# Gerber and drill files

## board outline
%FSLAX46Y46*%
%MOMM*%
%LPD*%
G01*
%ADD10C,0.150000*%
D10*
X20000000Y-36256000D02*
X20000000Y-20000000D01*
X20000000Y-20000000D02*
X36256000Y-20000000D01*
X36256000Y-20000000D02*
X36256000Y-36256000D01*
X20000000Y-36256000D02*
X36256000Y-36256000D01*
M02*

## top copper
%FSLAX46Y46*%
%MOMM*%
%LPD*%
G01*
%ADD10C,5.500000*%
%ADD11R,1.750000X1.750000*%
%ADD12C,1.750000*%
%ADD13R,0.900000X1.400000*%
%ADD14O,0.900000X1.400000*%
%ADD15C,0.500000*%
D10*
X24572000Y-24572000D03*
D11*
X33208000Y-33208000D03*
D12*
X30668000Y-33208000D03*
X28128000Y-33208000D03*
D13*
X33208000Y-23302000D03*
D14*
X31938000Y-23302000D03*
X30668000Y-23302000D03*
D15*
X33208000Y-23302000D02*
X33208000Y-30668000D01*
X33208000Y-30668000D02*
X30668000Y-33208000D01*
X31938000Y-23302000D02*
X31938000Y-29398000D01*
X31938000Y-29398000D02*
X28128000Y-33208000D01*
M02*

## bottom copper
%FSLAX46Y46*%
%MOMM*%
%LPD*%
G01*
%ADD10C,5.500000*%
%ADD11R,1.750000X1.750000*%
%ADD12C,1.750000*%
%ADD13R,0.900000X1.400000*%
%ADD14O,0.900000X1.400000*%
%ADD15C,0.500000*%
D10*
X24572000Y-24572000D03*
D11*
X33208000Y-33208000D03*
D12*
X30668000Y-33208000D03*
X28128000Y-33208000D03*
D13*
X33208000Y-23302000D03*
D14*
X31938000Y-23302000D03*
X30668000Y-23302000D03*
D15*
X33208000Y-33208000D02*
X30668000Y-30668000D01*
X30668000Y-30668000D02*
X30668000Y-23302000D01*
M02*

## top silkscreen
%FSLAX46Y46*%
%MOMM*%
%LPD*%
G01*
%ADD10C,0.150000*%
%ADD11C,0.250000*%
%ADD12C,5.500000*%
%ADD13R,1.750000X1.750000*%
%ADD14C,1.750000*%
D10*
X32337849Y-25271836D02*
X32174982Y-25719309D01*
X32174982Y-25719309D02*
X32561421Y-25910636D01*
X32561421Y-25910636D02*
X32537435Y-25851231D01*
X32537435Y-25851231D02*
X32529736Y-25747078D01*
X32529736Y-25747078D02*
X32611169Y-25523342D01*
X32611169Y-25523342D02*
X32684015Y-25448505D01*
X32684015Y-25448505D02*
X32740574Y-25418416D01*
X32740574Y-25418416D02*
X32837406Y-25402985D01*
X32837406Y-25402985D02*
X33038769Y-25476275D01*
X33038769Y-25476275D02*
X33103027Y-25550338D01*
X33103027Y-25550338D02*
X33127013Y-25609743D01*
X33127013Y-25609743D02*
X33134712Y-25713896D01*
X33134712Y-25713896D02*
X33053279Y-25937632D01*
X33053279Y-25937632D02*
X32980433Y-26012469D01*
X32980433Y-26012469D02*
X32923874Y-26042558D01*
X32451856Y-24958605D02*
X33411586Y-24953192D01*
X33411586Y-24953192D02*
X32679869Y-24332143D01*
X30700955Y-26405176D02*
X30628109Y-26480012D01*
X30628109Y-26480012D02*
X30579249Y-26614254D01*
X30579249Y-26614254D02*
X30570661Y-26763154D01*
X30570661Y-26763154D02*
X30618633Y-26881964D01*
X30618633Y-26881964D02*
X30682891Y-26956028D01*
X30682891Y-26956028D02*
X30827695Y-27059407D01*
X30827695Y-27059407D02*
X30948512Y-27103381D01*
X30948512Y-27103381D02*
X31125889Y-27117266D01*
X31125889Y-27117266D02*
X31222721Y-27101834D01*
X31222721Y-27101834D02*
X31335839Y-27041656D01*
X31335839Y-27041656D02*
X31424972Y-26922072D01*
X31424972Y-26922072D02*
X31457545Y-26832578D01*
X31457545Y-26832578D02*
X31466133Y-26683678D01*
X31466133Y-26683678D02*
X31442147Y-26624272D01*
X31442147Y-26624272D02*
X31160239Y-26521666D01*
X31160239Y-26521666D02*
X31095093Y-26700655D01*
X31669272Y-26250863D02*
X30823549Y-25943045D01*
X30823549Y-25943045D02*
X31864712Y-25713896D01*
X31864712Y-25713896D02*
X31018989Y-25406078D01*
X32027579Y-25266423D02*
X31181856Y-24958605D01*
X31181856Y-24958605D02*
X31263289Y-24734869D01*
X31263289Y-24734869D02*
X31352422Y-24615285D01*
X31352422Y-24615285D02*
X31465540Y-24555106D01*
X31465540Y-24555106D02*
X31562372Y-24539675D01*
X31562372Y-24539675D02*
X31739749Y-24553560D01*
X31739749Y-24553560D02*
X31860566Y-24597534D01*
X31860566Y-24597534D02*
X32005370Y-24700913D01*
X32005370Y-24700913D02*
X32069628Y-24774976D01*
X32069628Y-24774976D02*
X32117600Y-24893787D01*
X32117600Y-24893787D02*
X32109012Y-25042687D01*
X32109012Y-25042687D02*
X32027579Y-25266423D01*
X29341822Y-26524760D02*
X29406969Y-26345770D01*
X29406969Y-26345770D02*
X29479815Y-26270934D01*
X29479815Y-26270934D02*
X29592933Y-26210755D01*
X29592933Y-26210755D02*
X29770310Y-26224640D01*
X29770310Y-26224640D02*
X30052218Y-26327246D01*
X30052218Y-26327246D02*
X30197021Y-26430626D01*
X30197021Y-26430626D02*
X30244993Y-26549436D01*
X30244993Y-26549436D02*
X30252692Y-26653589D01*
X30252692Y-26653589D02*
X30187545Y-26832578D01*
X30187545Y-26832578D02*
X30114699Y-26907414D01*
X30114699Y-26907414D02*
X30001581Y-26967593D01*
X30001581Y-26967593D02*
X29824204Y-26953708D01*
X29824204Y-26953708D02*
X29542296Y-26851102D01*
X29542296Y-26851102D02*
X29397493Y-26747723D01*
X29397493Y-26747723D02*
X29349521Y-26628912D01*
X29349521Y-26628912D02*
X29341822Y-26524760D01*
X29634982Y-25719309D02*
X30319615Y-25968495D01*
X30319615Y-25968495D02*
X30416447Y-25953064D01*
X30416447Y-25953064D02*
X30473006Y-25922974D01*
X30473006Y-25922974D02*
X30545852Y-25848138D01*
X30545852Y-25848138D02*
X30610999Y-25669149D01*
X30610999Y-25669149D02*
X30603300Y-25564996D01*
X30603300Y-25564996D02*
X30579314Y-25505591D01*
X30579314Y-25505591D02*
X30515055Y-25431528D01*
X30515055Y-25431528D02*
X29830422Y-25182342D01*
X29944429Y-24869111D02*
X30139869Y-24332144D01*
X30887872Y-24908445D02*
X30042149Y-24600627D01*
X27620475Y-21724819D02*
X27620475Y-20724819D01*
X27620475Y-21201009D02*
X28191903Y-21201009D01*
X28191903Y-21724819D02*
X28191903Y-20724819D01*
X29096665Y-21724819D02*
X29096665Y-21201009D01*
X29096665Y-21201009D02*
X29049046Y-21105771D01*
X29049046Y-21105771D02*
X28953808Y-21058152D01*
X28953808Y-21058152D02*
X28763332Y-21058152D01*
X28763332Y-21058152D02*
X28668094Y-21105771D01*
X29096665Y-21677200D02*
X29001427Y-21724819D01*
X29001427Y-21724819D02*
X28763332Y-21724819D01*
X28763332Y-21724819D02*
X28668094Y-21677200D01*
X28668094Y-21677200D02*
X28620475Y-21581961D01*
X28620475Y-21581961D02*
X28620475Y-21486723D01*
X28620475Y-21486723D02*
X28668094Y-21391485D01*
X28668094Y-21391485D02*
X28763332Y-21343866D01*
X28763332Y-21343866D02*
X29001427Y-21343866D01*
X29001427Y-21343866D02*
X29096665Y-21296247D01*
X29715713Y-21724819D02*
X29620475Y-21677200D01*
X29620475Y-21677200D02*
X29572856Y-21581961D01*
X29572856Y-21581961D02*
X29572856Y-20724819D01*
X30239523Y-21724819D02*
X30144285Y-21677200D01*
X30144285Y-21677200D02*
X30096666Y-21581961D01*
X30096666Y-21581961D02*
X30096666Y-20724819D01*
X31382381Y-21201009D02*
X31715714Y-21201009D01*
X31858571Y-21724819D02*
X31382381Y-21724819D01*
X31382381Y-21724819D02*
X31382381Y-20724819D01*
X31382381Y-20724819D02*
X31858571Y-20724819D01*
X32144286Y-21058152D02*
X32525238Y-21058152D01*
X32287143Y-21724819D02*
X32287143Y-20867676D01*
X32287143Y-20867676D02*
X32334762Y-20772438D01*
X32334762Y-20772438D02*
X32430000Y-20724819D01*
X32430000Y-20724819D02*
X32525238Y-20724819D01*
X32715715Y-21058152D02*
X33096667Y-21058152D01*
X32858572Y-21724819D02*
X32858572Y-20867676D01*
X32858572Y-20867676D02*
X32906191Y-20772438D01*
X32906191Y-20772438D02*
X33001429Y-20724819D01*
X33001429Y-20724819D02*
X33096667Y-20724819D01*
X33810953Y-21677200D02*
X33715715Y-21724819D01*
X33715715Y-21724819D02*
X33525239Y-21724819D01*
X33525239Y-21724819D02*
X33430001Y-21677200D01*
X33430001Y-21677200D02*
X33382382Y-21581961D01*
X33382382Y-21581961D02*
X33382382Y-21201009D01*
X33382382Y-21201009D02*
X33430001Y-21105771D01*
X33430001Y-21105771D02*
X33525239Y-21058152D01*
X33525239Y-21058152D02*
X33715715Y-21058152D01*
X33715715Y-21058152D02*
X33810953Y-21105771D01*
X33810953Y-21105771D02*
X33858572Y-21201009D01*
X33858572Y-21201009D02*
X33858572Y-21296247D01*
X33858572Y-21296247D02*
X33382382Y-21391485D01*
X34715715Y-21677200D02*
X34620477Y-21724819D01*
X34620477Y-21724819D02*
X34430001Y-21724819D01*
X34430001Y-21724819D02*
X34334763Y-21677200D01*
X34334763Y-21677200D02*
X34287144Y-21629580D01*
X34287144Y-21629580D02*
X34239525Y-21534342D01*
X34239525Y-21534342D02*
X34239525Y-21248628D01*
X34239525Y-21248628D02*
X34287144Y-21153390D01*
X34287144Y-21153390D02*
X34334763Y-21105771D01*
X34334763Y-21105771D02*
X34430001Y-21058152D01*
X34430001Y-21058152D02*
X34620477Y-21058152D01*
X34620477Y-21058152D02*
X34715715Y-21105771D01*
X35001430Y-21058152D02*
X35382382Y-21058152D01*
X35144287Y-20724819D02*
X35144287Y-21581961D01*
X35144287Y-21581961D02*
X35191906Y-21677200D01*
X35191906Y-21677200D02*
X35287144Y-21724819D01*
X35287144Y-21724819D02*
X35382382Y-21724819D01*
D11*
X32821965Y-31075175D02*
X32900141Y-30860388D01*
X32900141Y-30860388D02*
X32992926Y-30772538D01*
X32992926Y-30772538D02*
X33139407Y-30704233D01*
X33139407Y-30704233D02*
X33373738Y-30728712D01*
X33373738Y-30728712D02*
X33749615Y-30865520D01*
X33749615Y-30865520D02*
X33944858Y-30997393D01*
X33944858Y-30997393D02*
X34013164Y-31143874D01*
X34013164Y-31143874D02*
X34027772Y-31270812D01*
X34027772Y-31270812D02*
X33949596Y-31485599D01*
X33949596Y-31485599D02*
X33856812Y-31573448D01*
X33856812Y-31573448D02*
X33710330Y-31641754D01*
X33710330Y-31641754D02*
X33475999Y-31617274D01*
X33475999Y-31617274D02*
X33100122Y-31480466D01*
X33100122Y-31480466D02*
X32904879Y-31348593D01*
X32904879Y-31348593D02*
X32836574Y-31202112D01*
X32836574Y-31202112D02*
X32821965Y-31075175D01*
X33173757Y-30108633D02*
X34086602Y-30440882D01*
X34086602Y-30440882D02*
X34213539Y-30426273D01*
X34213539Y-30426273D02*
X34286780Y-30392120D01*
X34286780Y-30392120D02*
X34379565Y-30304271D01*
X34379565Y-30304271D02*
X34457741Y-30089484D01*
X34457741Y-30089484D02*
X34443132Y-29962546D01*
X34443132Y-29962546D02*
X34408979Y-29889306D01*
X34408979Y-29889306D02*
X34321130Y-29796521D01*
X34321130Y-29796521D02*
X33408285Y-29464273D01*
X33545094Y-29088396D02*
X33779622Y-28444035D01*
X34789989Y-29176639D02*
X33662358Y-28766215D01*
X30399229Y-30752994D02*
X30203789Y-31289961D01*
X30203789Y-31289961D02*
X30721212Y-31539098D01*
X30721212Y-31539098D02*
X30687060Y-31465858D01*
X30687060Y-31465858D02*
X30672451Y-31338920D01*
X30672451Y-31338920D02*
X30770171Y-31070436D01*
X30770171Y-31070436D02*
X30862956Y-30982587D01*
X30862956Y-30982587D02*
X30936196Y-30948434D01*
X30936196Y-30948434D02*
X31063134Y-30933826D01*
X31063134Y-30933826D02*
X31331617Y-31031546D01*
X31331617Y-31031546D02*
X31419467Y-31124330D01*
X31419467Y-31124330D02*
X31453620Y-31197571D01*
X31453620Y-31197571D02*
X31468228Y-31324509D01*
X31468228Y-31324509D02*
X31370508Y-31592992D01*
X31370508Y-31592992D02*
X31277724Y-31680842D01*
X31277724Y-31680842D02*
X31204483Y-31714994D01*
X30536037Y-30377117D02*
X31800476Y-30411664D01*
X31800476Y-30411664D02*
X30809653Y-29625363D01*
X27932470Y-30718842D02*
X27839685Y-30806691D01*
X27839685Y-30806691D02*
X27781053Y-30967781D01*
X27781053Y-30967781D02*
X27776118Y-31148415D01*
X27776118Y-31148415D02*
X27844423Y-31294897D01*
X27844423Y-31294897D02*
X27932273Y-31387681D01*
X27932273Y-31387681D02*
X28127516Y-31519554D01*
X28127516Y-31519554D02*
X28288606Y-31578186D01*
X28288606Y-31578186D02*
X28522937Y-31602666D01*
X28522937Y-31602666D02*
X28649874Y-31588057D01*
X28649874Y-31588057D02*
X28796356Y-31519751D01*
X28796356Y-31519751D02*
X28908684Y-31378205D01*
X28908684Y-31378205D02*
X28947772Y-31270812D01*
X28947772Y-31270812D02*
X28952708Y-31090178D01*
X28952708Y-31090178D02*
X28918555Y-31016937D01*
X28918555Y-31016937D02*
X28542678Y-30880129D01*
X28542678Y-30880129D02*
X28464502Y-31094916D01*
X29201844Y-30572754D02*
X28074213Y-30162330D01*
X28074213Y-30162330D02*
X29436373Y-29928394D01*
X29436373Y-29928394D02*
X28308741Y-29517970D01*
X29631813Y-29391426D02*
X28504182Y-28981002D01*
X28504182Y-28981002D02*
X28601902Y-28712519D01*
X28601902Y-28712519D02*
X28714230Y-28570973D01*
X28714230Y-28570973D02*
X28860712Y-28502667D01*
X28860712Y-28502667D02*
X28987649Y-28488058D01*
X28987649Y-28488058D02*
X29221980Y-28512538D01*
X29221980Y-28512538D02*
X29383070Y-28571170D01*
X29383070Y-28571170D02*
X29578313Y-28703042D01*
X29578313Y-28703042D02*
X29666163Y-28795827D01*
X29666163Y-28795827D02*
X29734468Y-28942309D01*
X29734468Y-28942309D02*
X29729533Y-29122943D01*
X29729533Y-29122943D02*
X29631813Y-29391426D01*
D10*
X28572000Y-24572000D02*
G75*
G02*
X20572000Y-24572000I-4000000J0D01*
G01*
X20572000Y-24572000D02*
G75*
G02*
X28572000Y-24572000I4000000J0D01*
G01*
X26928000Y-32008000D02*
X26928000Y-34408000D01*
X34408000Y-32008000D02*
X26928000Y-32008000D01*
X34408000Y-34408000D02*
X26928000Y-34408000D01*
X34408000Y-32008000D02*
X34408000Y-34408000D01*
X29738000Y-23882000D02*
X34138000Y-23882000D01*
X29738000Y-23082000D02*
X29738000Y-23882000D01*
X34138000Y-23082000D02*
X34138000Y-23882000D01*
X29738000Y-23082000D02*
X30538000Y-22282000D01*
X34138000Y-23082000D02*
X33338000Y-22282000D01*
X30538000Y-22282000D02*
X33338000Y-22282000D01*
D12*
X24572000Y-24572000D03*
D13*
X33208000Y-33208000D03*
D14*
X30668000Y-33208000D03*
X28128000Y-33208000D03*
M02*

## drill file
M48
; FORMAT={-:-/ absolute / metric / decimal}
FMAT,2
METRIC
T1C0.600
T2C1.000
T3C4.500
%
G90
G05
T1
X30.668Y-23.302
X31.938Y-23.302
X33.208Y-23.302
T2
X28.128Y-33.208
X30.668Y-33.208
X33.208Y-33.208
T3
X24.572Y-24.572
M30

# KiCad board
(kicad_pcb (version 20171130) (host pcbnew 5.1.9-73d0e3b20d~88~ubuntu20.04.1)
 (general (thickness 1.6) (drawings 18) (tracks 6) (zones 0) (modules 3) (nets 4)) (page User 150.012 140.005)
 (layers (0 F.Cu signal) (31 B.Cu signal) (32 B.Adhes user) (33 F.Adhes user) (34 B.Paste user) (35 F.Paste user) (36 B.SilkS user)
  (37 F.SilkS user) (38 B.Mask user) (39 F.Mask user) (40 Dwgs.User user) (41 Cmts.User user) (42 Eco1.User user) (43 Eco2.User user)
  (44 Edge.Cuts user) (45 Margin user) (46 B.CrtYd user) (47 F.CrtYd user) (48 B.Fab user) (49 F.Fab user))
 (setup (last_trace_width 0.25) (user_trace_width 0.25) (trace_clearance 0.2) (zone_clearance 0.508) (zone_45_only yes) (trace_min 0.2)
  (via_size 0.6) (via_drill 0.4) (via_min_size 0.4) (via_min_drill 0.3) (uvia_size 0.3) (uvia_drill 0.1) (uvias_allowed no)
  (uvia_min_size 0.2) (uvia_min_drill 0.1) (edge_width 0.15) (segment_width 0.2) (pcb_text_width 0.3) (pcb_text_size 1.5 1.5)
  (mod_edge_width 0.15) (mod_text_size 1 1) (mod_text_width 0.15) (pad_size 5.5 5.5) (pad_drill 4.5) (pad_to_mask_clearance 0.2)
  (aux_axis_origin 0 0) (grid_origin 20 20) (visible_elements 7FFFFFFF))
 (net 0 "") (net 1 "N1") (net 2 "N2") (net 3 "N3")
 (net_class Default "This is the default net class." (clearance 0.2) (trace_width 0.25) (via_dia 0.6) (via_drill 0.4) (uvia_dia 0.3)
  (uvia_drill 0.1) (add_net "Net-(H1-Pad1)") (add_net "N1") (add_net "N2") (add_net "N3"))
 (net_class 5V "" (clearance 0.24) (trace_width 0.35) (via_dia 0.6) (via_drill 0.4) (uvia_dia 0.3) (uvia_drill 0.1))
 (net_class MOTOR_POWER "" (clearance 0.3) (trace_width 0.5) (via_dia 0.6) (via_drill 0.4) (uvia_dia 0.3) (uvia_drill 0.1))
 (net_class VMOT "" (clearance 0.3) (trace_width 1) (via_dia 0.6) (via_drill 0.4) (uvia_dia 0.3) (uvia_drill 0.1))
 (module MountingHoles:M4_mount (layer F.Cu) (at 24.572 24.572)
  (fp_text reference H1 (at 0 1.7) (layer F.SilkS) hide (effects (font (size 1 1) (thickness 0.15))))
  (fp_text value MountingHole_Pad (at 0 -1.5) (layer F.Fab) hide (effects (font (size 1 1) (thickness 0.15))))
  (fp_circle (center 0 0) (end 4 0) (layer F.SilkS) (width 0.15))
  (pad 1 thru_hole circle (at 0 0) (size 5.5 5.5) (drill 4.5) (layers *.Cu *.Mask F.SilkS) (clearance 1.5)))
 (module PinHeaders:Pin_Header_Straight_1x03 (layer F.Cu) (at 33.208 33.208 270)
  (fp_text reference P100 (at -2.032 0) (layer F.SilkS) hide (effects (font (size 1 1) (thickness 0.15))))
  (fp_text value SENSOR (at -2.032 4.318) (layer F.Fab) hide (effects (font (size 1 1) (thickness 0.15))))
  (fp_line (start -1.2 6.28) (end 1.2 6.28) (layer F.SilkS) (width 0.15))
  (fp_line (start -1.2 -1.2) (end -1.2 6.28) (layer F.SilkS) (width 0.15))
  (fp_line (start 1.2 -1.2) (end 1.2 6.28) (layer F.SilkS) (width 0.15))
  (fp_line (start -1.2 -1.2) (end 1.2 -1.2) (layer F.SilkS) (width 0.15))
  (pad 1 thru_hole rect (at 0 0 270) (size 1.75 1.75) (drill 1) (layers *.Cu *.Mask F.SilkS) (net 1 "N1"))
  (pad 2 thru_hole circle (at 0 2.54 270) (size 1.75 1.75) (drill 1) (layers *.Cu *.Mask F.SilkS) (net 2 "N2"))
  (pad 3 thru_hole circle (at 0 5.08 270) (size 1.75 1.75) (drill 1) (layers *.Cu *.Mask F.SilkS) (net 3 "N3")))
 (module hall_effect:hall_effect (layer B.Cu) (at 31.938 23.302 180)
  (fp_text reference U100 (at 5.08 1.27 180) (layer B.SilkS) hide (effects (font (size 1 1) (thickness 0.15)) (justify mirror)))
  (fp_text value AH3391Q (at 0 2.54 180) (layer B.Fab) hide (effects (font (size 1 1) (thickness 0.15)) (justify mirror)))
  (fp_line (start 2.2 -0.58) (end -2.2 -0.58) (layer F.SilkS) (width 0.15))
  (fp_line (start 2.2 0.22) (end 2.2 -0.58) (layer F.SilkS) (width 0.15))
  (fp_line (start -2.2 0.22) (end -2.2 -0.58) (layer F.SilkS) (width 0.15))
  (fp_line (start 2.2 0.22) (end 1.4 1.02) (layer F.SilkS) (width 0.15))
  (fp_line (start -2.2 0.22) (end -1.4 1.02) (layer F.SilkS) (width 0.15))
  (fp_line (start 1.4 1.02) (end -1.4 1.02) (layer F.SilkS) (width 0.15))
  (pad 1 thru_hole rect (at -1.27 0 180) (size 0.9 1.4) (drill 0.6) (layers *.Cu *.Mask) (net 2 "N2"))
  (pad 2 thru_hole oval (at 0 0 180) (size 0.9 1.4) (drill 0.6) (layers *.Cu *.Mask) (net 3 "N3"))
  (pad 3 thru_hole oval (at 1.27 0 180) (size 0.9 1.4) (drill 0.6) (layers *.Cu *.Mask) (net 1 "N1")))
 (gr_line (start 20 36.256) (end 20 20) (angle 90) (layer Edge.Cuts) (width 0.15))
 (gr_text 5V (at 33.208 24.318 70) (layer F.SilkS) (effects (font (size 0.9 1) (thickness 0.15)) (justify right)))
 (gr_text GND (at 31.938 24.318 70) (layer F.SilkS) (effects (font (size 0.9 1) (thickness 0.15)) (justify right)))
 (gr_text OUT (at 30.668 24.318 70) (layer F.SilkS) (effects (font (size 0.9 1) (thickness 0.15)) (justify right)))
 (gr_line (start 20 20) (end 36.256 20) (angle 90) (layer Edge.Cuts) (width 0.15))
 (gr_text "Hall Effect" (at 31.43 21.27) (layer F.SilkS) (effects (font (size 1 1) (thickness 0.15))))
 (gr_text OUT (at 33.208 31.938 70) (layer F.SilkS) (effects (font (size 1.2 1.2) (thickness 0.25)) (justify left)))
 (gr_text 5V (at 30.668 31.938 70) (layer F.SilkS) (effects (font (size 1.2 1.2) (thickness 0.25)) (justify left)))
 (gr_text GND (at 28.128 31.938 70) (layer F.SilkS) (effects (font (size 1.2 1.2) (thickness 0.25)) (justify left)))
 (gr_line (start 36.256 20) (end 36.256 36.256) (angle 90) (layer Edge.Cuts) (width 0.15))
 (gr_line (start 20 36.256) (end 36.256 36.256) (angle 90) (layer Edge.Cuts) (width 0.15))
 (segment (start 33.208 33.208) (end 30.668 30.668) (width 0.5) (layer B.Cu) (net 1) (status 10))
 (segment (start 30.668 30.668) (end 30.668 23.302) (width 0.5) (layer B.Cu) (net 1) (status 20))
 (segment (start 33.208 23.302) (end 33.208 30.668) (width 0.5) (layer F.Cu) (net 2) (status 10))
 (segment (start 33.208 30.668) (end 30.668 33.208) (width 0.5) (layer F.Cu) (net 2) (status 20))
 (segment (start 31.938 23.302) (end 31.938 29.398) (width 0.5) (layer F.Cu) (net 3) (status 10))
 (segment (start 31.938 29.398) (end 28.128 33.208) (width 0.5) (layer F.Cu) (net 3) (status 20)))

